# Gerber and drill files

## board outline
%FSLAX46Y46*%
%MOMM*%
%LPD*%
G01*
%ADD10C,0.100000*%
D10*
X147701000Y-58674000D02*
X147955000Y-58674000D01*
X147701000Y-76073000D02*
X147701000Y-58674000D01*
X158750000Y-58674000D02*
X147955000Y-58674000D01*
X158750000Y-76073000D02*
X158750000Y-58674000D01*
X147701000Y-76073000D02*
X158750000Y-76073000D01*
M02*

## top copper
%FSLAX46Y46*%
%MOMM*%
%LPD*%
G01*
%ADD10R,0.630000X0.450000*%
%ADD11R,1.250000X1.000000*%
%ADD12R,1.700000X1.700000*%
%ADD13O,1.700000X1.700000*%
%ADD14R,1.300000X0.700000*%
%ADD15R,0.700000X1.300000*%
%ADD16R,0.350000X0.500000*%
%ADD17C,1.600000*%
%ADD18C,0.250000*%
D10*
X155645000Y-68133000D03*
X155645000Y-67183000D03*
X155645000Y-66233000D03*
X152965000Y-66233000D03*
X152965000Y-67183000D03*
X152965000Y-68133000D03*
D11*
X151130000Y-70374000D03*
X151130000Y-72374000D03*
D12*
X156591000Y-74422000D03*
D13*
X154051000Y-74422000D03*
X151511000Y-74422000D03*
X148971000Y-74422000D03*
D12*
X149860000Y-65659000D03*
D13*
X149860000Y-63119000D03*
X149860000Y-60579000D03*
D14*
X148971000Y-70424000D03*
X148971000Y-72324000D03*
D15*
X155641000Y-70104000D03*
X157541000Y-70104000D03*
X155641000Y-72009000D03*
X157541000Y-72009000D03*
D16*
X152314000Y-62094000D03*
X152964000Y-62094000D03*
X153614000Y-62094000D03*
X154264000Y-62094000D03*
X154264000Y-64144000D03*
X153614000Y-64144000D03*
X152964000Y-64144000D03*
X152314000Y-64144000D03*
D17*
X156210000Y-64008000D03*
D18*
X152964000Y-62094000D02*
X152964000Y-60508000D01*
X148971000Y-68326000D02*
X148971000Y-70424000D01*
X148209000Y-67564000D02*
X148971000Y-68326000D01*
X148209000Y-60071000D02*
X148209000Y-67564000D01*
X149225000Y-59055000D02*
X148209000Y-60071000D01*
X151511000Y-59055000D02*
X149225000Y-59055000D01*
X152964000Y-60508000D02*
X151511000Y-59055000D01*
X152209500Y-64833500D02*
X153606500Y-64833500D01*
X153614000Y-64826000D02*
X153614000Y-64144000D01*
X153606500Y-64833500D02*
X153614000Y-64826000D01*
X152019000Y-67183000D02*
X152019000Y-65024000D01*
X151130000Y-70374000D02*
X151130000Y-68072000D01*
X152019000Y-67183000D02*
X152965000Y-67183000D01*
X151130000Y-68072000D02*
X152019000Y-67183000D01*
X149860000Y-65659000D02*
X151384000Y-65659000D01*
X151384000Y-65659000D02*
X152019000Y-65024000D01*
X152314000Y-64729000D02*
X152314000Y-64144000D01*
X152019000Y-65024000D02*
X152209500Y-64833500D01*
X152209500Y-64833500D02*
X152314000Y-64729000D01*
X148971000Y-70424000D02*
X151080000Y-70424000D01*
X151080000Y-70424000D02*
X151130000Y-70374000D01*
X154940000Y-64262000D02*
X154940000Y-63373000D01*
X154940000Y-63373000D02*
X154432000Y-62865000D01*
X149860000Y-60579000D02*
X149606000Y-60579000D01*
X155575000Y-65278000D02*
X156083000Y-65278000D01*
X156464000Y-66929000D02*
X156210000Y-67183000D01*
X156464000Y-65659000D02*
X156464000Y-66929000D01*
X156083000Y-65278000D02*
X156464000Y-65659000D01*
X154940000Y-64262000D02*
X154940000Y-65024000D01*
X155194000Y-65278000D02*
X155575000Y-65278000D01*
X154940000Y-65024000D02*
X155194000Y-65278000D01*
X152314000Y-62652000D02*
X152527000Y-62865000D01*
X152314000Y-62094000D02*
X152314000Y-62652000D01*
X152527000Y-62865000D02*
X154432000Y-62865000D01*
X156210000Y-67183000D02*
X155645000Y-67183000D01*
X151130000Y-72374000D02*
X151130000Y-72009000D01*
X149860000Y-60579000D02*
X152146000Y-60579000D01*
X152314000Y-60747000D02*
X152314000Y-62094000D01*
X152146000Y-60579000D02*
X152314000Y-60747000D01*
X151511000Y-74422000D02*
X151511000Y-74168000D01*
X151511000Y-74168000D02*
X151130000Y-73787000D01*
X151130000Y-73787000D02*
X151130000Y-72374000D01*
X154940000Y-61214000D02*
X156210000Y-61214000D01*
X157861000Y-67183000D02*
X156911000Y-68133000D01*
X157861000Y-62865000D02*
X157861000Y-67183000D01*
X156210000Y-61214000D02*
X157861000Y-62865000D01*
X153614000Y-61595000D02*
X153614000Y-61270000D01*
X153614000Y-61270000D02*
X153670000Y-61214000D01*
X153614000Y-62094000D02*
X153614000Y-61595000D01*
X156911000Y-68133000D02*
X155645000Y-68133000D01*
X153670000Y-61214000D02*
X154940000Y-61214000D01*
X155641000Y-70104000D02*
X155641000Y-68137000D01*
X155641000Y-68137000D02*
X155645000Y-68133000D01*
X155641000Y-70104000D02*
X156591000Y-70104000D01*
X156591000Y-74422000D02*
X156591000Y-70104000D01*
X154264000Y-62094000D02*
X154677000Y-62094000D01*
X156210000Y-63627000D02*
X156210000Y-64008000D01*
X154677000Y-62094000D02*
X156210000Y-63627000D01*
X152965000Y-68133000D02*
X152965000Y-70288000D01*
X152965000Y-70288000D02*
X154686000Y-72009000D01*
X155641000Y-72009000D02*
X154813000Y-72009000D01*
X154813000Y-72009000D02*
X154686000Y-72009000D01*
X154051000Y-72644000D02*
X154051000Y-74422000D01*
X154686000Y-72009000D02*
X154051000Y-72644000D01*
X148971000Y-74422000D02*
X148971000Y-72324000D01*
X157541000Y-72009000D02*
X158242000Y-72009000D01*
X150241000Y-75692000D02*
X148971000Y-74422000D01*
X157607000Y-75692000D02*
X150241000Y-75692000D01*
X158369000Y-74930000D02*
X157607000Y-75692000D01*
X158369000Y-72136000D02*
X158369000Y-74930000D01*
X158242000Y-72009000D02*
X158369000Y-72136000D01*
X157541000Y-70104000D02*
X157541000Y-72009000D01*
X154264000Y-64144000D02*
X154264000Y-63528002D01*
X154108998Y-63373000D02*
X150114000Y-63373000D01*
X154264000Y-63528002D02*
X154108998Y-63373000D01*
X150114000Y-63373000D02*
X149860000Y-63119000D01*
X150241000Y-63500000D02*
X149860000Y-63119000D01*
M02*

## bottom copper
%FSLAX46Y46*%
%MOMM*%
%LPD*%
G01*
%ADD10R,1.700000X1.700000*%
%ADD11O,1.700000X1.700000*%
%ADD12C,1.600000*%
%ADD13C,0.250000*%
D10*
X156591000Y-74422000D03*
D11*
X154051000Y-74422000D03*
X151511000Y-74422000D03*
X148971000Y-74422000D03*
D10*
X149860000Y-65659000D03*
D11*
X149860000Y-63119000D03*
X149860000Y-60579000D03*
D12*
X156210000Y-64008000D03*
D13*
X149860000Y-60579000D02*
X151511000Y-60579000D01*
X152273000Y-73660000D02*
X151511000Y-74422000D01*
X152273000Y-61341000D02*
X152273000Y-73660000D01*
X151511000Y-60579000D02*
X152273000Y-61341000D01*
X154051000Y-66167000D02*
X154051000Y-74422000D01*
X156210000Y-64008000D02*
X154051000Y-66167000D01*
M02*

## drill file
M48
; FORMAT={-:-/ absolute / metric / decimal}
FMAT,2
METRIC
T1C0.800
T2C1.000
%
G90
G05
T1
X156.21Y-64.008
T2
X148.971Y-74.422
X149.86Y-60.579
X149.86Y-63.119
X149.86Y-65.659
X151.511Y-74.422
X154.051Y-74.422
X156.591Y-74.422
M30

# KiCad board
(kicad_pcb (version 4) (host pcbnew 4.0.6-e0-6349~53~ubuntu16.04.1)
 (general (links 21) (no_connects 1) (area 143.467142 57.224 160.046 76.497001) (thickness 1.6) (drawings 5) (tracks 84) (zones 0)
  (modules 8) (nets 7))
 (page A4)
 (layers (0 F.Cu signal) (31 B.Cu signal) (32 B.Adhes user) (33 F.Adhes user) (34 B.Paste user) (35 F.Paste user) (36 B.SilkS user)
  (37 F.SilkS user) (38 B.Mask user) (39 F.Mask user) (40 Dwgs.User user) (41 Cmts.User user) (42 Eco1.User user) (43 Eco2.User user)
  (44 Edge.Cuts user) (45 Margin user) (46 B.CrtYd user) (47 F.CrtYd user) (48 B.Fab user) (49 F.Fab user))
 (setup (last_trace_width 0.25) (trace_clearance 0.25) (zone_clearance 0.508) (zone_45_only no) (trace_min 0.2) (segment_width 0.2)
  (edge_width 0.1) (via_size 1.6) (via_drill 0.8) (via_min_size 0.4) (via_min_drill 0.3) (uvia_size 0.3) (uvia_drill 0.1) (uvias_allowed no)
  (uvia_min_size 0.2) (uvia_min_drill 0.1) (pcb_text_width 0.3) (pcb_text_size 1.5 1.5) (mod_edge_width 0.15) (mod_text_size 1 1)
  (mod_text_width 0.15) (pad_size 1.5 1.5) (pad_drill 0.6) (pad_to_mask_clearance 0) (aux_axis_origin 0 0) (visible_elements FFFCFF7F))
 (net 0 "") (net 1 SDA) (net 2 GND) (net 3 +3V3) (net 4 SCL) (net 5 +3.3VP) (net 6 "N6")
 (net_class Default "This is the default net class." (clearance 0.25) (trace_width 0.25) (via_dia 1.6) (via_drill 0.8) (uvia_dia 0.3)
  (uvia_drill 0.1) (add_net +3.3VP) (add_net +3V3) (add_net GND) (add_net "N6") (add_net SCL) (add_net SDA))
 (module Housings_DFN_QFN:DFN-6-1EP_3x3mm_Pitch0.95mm (layer F.Cu) (at 154.305 67.183 180)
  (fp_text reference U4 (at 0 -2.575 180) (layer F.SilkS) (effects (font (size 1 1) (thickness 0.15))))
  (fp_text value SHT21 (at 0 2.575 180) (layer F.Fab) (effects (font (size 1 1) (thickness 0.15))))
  (pad 1 smd rect (at -1.34 -0.95 180) (size 0.63 0.45) (layers F.Cu F.Paste F.Mask) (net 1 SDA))
  (pad 2 smd rect (at -1.34 0 180) (size 0.63 0.45) (layers F.Cu F.Paste F.Mask) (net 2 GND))
  (pad 3 smd rect (at -1.34 0.95 180) (size 0.63 0.45) (layers F.Cu F.Paste F.Mask))
  (pad 4 smd rect (at 1.34 0.95 180) (size 0.63 0.45) (layers F.Cu F.Paste F.Mask))
  (pad 5 smd rect (at 1.34 0 180) (size 0.63 0.45) (layers F.Cu F.Paste F.Mask) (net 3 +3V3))
  (pad 6 smd rect (at 1.34 -0.95 180) (size 0.63 0.45) (layers F.Cu F.Paste F.Mask) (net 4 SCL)))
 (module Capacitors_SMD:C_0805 (layer F.Cu) (at 151.13 71.374 270)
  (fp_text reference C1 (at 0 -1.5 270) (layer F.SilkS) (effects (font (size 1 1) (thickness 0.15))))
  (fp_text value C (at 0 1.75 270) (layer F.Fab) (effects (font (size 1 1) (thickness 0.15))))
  (pad 1 smd rect (at -1 0 270) (size 1 1.25) (layers F.Cu F.Paste F.Mask) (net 3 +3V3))
  (pad 2 smd rect (at 1 0 270) (size 1 1.25) (layers F.Cu F.Paste F.Mask) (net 2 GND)))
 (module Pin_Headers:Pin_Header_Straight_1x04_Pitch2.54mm (layer F.Cu) (at 156.591 74.422 270)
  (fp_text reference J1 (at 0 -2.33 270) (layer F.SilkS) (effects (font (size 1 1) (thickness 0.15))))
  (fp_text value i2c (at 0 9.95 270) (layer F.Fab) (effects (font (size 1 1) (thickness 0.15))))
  (pad 1 thru_hole rect (at 0 0 270) (size 1.7 1.7) (drill 1) (layers *.Cu *.Mask) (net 1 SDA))
  (pad 2 thru_hole oval (at 0 2.54 270) (size 1.7 1.7) (drill 1) (layers *.Cu *.Mask) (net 4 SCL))
  (pad 3 thru_hole oval (at 0 5.08 270) (size 1.7 1.7) (drill 1) (layers *.Cu *.Mask) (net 2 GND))
  (pad 4 thru_hole oval (at 0 7.62 270) (size 1.7 1.7) (drill 1) (layers *.Cu *.Mask) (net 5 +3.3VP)))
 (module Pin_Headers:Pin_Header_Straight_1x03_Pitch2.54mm (layer F.Cu) (at 149.86 65.659 180)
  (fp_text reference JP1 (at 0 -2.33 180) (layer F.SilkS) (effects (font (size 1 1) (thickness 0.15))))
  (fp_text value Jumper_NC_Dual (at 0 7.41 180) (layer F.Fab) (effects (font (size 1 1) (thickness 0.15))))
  (pad 1 thru_hole rect (at 0 0 180) (size 1.7 1.7) (drill 1) (layers *.Cu *.Mask) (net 3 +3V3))
  (pad 2 thru_hole oval (at 0 2.54 180) (size 1.7 1.7) (drill 1) (layers *.Cu *.Mask) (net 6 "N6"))
  (pad 3 thru_hole oval (at 0 5.08 180) (size 1.7 1.7) (drill 1) (layers *.Cu *.Mask) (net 2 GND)))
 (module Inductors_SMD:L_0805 (layer F.Cu) (at 148.971 71.374 270)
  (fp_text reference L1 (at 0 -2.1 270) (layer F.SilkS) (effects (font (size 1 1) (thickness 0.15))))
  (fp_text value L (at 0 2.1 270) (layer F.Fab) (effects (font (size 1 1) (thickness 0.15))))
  (pad 1 smd rect (at -0.95 0 270) (size 0.7 1.3) (layers F.Cu F.Paste F.Mask) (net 3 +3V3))
  (pad 2 smd rect (at 0.95 0 270) (size 0.7 1.3) (layers F.Cu F.Paste F.Mask) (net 5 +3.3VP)))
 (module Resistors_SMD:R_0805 (layer F.Cu) (at 156.591 70.104)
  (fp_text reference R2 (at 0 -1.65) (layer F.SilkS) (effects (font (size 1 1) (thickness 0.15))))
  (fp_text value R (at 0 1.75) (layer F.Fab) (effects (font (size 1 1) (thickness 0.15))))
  (pad 1 smd rect (at -0.95 0) (size 0.7 1.3) (layers F.Cu F.Paste F.Mask) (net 1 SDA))
  (pad 2 smd rect (at 0.95 0) (size 0.7 1.3) (layers F.Cu F.Paste F.Mask) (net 5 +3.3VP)))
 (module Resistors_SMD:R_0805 (layer F.Cu) (at 156.591 72.009)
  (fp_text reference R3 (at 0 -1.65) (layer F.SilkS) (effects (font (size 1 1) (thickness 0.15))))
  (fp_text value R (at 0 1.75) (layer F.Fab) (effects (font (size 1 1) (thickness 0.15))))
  (pad 1 smd rect (at -0.95 0) (size 0.7 1.3) (layers F.Cu F.Paste F.Mask) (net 4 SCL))
  (pad 2 smd rect (at 0.95 0) (size 0.7 1.3) (layers F.Cu F.Paste F.Mask) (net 5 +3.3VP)))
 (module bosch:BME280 (layer F.Cu) (at 153.289 63.119 90)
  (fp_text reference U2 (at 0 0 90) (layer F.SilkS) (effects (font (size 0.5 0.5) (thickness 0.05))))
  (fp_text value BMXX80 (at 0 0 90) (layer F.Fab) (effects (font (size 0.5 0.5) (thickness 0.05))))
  (pad 1 smd rect (at 1.025 -0.975 90) (size 0.5 0.35) (layers F.Cu F.Paste F.Mask) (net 2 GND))
  (pad 2 smd rect (at 1.025 -0.325 90) (size 0.5 0.35) (layers F.Cu F.Paste F.Mask) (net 3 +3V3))
  (pad 3 smd rect (at 1.025 0.325 90) (size 0.5 0.35) (layers F.Cu F.Paste F.Mask) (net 1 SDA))
  (pad 4 smd rect (at 1.025 0.975 90) (size 0.5 0.35) (layers F.Cu F.Paste F.Mask) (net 4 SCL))
  (pad 5 smd rect (at -1.025 0.975 90) (size 0.5 0.35) (layers F.Cu F.Paste F.Mask) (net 6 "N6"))
  (pad 6 smd rect (at -1.025 0.325 90) (size 0.5 0.35) (layers F.Cu F.Paste F.Mask) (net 3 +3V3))
  (pad 7 smd rect (at -1.025 -0.325 90) (size 0.5 0.35) (layers F.Cu F.Paste F.Mask) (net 2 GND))
  (pad 8 smd rect (at -1.025 -0.975 90) (size 0.5 0.35) (layers F.Cu F.Paste F.Mask) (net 3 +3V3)))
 (gr_line (start 147.701 58.674) (end 147.955 58.674) (angle 90) (layer Edge.Cuts) (width 0.1))
 (gr_line (start 147.701 76.073) (end 147.701 58.674) (angle 90) (layer Edge.Cuts) (width 0.1))
 (gr_line (start 158.75 58.674) (end 147.955 58.674) (angle 90) (layer Edge.Cuts) (width 0.1))
 (gr_line (start 158.75 76.073) (end 158.75 58.674) (angle 90) (layer Edge.Cuts) (width 0.1))
 (gr_line (start 147.701 76.073) (end 158.75 76.073) (angle 90) (layer Edge.Cuts) (width 0.1))
 (segment (start 152.964 62.094) (end 152.964 60.508) (width 0.25) (layer F.Cu) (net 3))
 (segment (start 148.971 68.326) (end 148.971 70.424) (width 0.25) (layer F.Cu) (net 3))
 (segment (start 148.209 67.564) (end 148.971 68.326) (width 0.25) (layer F.Cu) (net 3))
 (segment (start 148.209 60.071) (end 148.209 67.564) (width 0.25) (layer F.Cu) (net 3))
 (segment (start 149.225 59.055) (end 148.209 60.071) (width 0.25) (layer F.Cu) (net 3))
 (segment (start 151.511 59.055) (end 149.225 59.055) (width 0.25) (layer F.Cu) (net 3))
 (segment (start 152.964 60.508) (end 151.511 59.055) (width 0.25) (layer F.Cu) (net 3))
 (segment (start 152.2095 64.8335) (end 153.6065 64.8335) (width 0.25) (layer F.Cu) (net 3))
 (segment (start 153.614 64.826) (end 153.614 64.144) (width 0.25) (layer F.Cu) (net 3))
 (segment (start 153.6065 64.8335) (end 153.614 64.826) (width 0.25) (layer F.Cu) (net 3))
 (segment (start 152.019 67.183) (end 152.019 65.024) (width 0.25) (layer F.Cu) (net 3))
 (segment (start 151.13 70.374) (end 151.13 68.072) (width 0.25) (layer F.Cu) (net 3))
 (segment (start 152.019 67.183) (end 152.965 67.183) (width 0.25) (layer F.Cu) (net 3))
 (segment (start 151.13 68.072) (end 152.019 67.183) (width 0.25) (layer F.Cu) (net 3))
 (segment (start 149.86 65.659) (end 151.384 65.659) (width 0.25) (layer F.Cu) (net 3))
 (segment (start 151.384 65.659) (end 152.019 65.024) (width 0.25) (layer F.Cu) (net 3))
 (segment (start 152.314 64.729) (end 152.314 64.144) (width 0.25) (layer F.Cu) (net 3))
 (segment (start 152.019 65.024) (end 152.2095 64.8335) (width 0.25) (layer F.Cu) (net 3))
 (segment (start 152.2095 64.8335) (end 152.314 64.729) (width 0.25) (layer F.Cu) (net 3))
 (segment (start 148.971 70.424) (end 151.08 70.424) (width 0.25) (layer F.Cu) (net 3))
 (segment (start 151.08 70.424) (end 151.13 70.374) (width 0.25) (layer F.Cu) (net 3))
 (segment (start 149.86 60.579) (end 151.511 60.579) (width 0.25) (layer B.Cu) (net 2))
 (segment (start 152.273 73.66) (end 151.511 74.422) (width 0.25) (layer B.Cu) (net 2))
 (segment (start 152.273 61.341) (end 152.273 73.66) (width 0.25) (layer B.Cu) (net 2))
 (segment (start 151.511 60.579) (end 152.273 61.341) (width 0.25) (layer B.Cu) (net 2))
 (segment (start 154.94 64.262) (end 154.94 63.373) (width 0.25) (layer F.Cu) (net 2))
 (segment (start 154.94 63.373) (end 154.432 62.865) (width 0.25) (layer F.Cu) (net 2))
 (segment (start 149.86 60.579) (end 149.606 60.579) (width 0.25) (layer F.Cu) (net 2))
 (segment (start 155.575 65.278) (end 156.083 65.278) (width 0.25) (layer F.Cu) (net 2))
 (segment (start 156.464 66.929) (end 156.21 67.183) (width 0.25) (layer F.Cu) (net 2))
 (segment (start 156.464 65.659) (end 156.464 66.929) (width 0.25) (layer F.Cu) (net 2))
 (segment (start 156.083 65.278) (end 156.464 65.659) (width 0.25) (layer F.Cu) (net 2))
 (segment (start 154.94 64.262) (end 154.94 65.024) (width 0.25) (layer F.Cu) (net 2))
 (segment (start 155.194 65.278) (end 155.575 65.278) (width 0.25) (layer F.Cu) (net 2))
 (segment (start 154.94 65.024) (end 155.194 65.278) (width 0.25) (layer F.Cu) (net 2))
 (segment (start 152.314 62.652) (end 152.527 62.865) (width 0.25) (layer F.Cu) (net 2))
 (segment (start 152.314 62.094) (end 152.314 62.652) (width 0.25) (layer F.Cu) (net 2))
 (segment (start 152.527 62.865) (end 154.432 62.865) (width 0.25) (layer F.Cu) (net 2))
 (segment (start 156.21 67.183) (end 155.645 67.183) (width 0.25) (layer F.Cu) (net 2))
 (segment (start 151.13 72.374) (end 151.13 72.009) (width 0.25) (layer F.Cu) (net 2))
 (segment (start 149.86 60.579) (end 152.146 60.579) (width 0.25) (layer F.Cu) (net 2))
 (segment (start 152.314 60.747) (end 152.314 62.094) (width 0.25) (layer F.Cu) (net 2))
 (segment (start 152.146 60.579) (end 152.314 60.747) (width 0.25) (layer F.Cu) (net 2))
 (segment (start 151.511 74.422) (end 151.511 74.168) (width 0.25) (layer F.Cu) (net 2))
 (segment (start 151.511 74.168) (end 151.13 73.787) (width 0.25) (layer F.Cu) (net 2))
 (segment (start 151.13 73.787) (end 151.13 72.374) (width 0.25) (layer F.Cu) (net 2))
 (segment (start 154.94 61.214) (end 156.21 61.214) (width 0.25) (layer F.Cu) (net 1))
 (segment (start 157.861 67.183) (end 156.911 68.133) (width 0.25) (layer F.Cu) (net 1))
 (segment (start 157.861 62.865) (end 157.861 67.183) (width 0.25) (layer F.Cu) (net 1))
 (segment (start 156.21 61.214) (end 157.861 62.865) (width 0.25) (layer F.Cu) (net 1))
 (segment (start 153.614 61.595) (end 153.614 61.27) (width 0.25) (layer F.Cu) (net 1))
 (segment (start 153.614 61.27) (end 153.67 61.214) (width 0.25) (layer F.Cu) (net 1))
 (segment (start 153.614 62.094) (end 153.614 61.595) (width 0.25) (layer F.Cu) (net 1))
 (segment (start 156.911 68.133) (end 155.645 68.133) (width 0.25) (layer F.Cu) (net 1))
 (segment (start 153.67 61.214) (end 154.94 61.214) (width 0.25) (layer F.Cu) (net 1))
 (segment (start 155.641 70.104) (end 155.641 68.137) (width 0.25) (layer F.Cu) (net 1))
 (segment (start 155.641 68.137) (end 155.645 68.133) (width 0.25) (layer F.Cu) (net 1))
 (segment (start 155.641 70.104) (end 156.591 70.104) (width 0.25) (layer F.Cu) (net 1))
 (segment (start 156.591 74.422) (end 156.591 70.104) (width 0.25) (layer F.Cu) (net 1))
 (segment (start 154.264 62.094) (end 154.677 62.094) (width 0.25) (layer F.Cu) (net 4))
 (segment (start 154.051 66.167) (end 154.051 74.422) (width 0.25) (layer B.Cu) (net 4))
 (segment (start 156.21 64.008) (end 154.051 66.167) (width 0.25) (layer B.Cu) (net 4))
 (via (at 156.21 64.008) (size 1.6) (drill 0.8) (layers F.Cu B.Cu) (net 4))
 (segment (start 156.21 63.627) (end 156.21 64.008) (width 0.25) (layer F.Cu) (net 4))
 (segment (start 154.677 62.094) (end 156.21 63.627) (width 0.25) (layer F.Cu) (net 4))
 (segment (start 152.965 68.133) (end 152.965 70.288) (width 0.25) (layer F.Cu) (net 4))
 (segment (start 152.965 70.288) (end 154.686 72.009) (width 0.25) (layer F.Cu) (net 4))
 (segment (start 155.641 72.009) (end 154.813 72.009) (width 0.25) (layer F.Cu) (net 4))
 (segment (start 154.813 72.009) (end 154.686 72.009) (width 0.25) (layer F.Cu) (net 4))
 (segment (start 154.051 72.644) (end 154.051 74.422) (width 0.25) (layer F.Cu) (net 4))
 (segment (start 154.686 72.009) (end 154.051 72.644) (width 0.25) (layer F.Cu) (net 4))
 (segment (start 148.971 74.422) (end 148.971 72.324) (width 0.25) (layer F.Cu) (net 5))
 (segment (start 157.541 72.009) (end 158.242 72.009) (width 0.25) (layer F.Cu) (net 5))
 (segment (start 150.241 75.692) (end 148.971 74.422) (width 0.25) (layer F.Cu) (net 5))
 (segment (start 157.607 75.692) (end 150.241 75.692) (width 0.25) (layer F.Cu) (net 5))
 (segment (start 158.369 74.93) (end 157.607 75.692) (width 0.25) (layer F.Cu) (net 5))
 (segment (start 158.369 72.136) (end 158.369 74.93) (width 0.25) (layer F.Cu) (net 5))
 (segment (start 158.242 72.009) (end 158.369 72.136) (width 0.25) (layer F.Cu) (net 5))
 (segment (start 157.541 70.104) (end 157.541 72.009) (width 0.25) (layer F.Cu) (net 5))
 (segment (start 154.264 64.144) (end 154.264 63.528002) (width 0.25) (layer F.Cu) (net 6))
 (segment (start 154.108998 63.373) (end 150.114 63.373) (width 0.25) (layer F.Cu) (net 6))
 (segment (start 154.264 63.528002) (end 154.108998 63.373) (width 0.25) (layer F.Cu) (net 6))
 (segment (start 150.114 63.373) (end 149.86 63.119) (width 0.25) (layer F.Cu) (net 6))
 (segment (start 150.241 63.5) (end 149.86 63.119) (width 0.25) (layer F.Cu) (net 6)))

